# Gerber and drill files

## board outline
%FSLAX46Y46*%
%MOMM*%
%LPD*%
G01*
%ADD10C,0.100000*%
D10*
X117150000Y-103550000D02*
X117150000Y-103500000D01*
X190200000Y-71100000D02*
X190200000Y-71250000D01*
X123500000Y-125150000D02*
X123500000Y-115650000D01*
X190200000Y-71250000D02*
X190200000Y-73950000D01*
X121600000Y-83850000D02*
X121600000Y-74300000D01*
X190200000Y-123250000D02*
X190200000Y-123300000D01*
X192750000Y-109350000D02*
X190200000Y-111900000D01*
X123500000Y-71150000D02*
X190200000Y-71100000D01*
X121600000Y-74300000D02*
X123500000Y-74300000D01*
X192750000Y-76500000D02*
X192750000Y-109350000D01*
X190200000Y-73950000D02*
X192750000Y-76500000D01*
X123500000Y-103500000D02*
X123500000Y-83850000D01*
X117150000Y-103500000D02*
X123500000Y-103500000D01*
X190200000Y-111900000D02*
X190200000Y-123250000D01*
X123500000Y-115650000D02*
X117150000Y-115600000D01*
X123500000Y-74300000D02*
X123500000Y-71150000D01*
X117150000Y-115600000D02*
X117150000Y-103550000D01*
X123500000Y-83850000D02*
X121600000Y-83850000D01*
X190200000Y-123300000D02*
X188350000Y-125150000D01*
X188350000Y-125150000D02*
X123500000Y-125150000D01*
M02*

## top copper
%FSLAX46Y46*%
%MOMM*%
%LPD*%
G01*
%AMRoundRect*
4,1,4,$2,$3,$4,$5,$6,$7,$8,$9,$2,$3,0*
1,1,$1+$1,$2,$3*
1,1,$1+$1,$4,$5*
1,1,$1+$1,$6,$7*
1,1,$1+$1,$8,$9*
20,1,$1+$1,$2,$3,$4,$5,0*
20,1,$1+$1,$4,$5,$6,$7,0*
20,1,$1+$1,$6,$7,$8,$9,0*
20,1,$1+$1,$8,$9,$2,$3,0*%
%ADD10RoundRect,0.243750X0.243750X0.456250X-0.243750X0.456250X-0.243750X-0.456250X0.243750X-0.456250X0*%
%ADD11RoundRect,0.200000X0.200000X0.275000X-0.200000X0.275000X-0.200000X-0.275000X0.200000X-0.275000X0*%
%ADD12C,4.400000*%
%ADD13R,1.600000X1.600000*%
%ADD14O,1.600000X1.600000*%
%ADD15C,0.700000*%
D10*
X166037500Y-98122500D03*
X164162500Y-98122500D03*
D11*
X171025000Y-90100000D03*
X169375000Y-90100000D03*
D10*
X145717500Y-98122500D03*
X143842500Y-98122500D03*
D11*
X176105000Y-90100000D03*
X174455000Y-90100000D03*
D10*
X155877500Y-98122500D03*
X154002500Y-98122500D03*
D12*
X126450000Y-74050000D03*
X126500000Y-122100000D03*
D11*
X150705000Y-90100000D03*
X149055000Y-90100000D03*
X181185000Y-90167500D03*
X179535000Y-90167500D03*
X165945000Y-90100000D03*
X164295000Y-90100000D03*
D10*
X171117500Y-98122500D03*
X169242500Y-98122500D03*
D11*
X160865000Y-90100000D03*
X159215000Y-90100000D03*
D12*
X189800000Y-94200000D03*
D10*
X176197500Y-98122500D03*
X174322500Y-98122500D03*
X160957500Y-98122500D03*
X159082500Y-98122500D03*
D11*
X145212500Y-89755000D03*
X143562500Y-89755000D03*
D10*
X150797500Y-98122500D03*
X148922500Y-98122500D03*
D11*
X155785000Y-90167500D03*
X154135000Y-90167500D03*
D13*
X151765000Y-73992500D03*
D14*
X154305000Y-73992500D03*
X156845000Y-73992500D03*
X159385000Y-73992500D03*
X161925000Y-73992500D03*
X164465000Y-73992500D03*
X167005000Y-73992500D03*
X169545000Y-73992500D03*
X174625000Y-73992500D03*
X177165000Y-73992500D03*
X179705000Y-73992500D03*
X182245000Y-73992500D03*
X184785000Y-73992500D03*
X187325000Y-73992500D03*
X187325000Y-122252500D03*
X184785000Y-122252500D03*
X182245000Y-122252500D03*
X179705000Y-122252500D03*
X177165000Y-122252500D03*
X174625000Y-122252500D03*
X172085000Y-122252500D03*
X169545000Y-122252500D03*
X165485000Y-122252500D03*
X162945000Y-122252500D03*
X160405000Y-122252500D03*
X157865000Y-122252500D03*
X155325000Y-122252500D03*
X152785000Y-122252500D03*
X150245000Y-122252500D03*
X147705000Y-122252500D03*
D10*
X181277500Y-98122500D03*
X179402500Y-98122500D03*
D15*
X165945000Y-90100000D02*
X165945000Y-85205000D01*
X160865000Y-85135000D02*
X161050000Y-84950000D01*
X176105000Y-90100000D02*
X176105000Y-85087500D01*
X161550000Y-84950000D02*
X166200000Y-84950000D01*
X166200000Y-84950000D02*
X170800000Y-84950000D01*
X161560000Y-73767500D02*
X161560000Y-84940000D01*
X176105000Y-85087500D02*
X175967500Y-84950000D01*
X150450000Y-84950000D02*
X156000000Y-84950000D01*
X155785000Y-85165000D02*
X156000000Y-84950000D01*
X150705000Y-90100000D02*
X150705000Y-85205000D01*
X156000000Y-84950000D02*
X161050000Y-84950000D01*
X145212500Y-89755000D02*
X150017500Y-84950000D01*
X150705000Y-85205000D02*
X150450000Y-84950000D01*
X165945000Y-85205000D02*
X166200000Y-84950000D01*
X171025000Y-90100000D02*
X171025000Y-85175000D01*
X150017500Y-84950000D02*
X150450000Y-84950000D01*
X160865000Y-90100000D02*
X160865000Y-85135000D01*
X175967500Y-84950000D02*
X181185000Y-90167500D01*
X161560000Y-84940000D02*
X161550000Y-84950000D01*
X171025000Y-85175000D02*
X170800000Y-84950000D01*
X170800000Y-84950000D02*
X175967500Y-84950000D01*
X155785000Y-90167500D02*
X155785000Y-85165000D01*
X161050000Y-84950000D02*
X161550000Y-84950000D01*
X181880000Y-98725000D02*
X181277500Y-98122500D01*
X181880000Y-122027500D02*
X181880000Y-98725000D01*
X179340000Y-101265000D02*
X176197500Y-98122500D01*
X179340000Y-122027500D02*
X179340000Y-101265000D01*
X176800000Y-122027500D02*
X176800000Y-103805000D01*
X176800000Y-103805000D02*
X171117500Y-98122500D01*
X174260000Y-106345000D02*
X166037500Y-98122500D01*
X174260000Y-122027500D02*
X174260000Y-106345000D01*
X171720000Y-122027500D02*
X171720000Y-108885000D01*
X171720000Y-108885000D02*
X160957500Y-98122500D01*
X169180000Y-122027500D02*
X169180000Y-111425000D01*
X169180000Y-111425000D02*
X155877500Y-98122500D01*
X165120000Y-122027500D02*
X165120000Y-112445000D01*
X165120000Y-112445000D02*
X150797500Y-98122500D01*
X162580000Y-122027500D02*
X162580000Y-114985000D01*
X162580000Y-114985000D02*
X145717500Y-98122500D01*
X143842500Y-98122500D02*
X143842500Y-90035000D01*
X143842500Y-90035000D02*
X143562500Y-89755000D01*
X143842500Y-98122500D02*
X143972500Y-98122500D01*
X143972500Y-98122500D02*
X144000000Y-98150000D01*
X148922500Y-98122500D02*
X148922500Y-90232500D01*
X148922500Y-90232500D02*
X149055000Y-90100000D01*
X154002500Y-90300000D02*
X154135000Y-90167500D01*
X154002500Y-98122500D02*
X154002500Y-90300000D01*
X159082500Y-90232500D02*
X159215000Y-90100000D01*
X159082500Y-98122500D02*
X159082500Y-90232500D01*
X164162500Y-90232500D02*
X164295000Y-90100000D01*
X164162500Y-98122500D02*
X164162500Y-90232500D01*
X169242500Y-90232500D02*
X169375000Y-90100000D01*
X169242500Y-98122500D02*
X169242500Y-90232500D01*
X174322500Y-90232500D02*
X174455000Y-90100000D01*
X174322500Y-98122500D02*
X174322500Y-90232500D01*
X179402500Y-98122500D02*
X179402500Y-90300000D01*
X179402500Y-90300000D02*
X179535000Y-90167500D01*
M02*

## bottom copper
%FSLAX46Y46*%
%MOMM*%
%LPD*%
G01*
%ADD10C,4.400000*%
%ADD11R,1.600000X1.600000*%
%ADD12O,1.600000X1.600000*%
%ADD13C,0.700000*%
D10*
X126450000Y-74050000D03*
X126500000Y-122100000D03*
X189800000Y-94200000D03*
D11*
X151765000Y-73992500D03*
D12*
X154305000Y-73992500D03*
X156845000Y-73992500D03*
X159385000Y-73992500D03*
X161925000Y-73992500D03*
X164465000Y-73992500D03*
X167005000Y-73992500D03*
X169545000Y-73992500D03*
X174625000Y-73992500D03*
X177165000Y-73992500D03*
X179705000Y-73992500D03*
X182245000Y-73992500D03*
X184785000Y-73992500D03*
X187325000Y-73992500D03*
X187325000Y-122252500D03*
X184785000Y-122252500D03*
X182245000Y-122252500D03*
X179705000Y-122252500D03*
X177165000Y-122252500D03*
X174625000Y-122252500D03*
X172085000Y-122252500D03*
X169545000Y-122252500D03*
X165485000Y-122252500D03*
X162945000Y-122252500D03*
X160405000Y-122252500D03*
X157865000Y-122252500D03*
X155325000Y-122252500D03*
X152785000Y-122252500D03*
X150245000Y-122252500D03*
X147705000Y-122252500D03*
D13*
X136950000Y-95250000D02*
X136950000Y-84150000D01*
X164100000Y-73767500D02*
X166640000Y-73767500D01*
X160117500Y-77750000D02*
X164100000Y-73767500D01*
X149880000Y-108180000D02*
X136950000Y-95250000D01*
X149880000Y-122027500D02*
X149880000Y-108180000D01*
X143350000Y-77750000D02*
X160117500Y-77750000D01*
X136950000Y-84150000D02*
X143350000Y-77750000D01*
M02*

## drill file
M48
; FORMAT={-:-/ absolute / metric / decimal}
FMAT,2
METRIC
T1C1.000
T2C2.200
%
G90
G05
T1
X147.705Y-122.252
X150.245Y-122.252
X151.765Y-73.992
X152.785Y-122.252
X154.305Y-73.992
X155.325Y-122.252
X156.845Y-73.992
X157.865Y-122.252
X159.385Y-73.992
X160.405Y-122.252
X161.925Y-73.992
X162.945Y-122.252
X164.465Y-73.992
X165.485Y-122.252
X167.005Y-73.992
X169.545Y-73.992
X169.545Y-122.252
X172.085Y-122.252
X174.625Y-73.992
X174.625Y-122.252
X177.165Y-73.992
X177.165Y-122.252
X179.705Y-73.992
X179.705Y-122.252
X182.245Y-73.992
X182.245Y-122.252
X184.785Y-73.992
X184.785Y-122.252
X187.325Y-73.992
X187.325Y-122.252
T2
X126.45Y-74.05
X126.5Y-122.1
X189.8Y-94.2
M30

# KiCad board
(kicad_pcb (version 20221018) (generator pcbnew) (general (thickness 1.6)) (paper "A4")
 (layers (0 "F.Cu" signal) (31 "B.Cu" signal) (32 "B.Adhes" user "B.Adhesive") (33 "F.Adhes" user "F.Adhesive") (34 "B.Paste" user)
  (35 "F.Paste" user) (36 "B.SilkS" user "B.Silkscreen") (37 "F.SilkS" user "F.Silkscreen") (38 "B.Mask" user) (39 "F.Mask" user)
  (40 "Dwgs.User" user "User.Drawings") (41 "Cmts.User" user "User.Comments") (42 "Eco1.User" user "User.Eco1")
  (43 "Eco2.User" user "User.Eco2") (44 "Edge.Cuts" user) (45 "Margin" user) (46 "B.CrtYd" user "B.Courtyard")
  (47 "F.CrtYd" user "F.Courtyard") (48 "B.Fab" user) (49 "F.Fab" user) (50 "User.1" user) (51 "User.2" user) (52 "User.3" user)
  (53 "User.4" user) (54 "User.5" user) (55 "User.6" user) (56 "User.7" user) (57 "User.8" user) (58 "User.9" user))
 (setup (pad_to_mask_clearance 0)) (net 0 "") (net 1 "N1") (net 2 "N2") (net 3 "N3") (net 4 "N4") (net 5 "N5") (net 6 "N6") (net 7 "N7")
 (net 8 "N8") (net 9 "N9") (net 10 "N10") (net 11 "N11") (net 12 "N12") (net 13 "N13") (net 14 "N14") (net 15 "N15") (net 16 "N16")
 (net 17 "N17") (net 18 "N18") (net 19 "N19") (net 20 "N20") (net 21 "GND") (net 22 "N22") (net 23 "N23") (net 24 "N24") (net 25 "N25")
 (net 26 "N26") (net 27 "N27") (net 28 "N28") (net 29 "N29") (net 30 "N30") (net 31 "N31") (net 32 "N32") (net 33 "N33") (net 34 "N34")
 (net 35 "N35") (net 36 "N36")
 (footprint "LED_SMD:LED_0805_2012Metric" (layer "F.Cu") (at 165.1 98.1225 180)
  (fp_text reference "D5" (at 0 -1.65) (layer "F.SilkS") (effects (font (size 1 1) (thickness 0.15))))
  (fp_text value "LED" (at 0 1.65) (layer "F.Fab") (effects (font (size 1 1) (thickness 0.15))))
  (pad "1" smd roundrect (at -0.9375 0 180) (size 0.975 1.4) (layers "F.Cu" "F.Paste" "F.Mask") (roundrect_rratio 0.25) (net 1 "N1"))
  (pad "2" smd roundrect (at 0.9375 0 180) (size 0.975 1.4) (layers "F.Cu" "F.Paste" "F.Mask") (roundrect_rratio 0.25) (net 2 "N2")))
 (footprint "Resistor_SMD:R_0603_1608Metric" (layer "F.Cu") (at 170.2 90.1 180)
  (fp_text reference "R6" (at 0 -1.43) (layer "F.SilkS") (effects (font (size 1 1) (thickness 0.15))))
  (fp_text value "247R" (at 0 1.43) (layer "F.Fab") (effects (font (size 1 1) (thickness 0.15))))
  (pad "1" smd roundrect (at -0.825 0 180) (size 0.8 0.95) (layers "F.Cu" "F.Paste" "F.Mask") (roundrect_rratio 0.25) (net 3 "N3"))
  (pad "2" smd roundrect (at 0.825 0 180) (size 0.8 0.95) (layers "F.Cu" "F.Paste" "F.Mask") (roundrect_rratio 0.25) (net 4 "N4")))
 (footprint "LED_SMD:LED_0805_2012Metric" (layer "F.Cu") (at 144.78 98.1225 180)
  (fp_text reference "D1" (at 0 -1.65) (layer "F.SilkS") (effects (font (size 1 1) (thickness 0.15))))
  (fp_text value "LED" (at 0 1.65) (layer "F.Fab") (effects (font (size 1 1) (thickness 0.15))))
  (pad "1" smd roundrect (at -0.9375 0 180) (size 0.975 1.4) (layers "F.Cu" "F.Paste" "F.Mask") (roundrect_rratio 0.25) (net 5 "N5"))
  (pad "2" smd roundrect (at 0.9375 0 180) (size 0.975 1.4) (layers "F.Cu" "F.Paste" "F.Mask") (roundrect_rratio 0.25) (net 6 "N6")))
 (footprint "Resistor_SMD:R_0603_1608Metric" (layer "F.Cu") (at 175.28 90.1 180)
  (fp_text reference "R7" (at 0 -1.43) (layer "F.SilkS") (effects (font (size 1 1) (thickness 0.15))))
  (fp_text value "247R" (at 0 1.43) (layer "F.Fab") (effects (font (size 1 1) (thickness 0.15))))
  (pad "1" smd roundrect (at -0.825 0 180) (size 0.8 0.95) (layers "F.Cu" "F.Paste" "F.Mask") (roundrect_rratio 0.25) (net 3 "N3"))
  (pad "2" smd roundrect (at 0.825 0 180) (size 0.8 0.95) (layers "F.Cu" "F.Paste" "F.Mask") (roundrect_rratio 0.25) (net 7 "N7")))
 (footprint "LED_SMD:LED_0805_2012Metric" (layer "F.Cu") (at 154.94 98.1225 180)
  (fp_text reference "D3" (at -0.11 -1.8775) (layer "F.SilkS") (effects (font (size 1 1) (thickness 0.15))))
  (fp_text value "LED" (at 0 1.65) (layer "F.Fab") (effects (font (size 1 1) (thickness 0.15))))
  (pad "1" smd roundrect (at -0.9375 0 180) (size 0.975 1.4) (layers "F.Cu" "F.Paste" "F.Mask") (roundrect_rratio 0.25) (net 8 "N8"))
  (pad "2" smd roundrect (at 0.9375 0 180) (size 0.975 1.4) (layers "F.Cu" "F.Paste" "F.Mask") (roundrect_rratio 0.25) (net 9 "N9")))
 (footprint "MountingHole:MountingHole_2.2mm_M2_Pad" (layer "F.Cu") (at 126.45 74.05)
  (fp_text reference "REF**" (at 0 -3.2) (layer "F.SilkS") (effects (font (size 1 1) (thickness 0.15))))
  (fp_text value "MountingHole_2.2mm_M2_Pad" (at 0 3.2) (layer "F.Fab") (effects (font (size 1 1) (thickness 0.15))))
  (pad "1" thru_hole circle (at 0 0) (size 4.4 4.4) (drill 2.2) (layers "*.Cu" "*.Mask")))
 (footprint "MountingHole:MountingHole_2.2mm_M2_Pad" (layer "F.Cu") (at 126.5 122.1)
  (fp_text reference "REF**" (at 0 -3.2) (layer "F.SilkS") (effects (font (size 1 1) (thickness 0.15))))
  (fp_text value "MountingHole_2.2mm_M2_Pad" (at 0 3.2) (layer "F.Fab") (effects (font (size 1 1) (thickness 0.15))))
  (pad "1" thru_hole circle (at 0 0) (size 4.4 4.4) (drill 2.2) (layers "*.Cu" "*.Mask")))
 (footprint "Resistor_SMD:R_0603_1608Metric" (layer "F.Cu") (at 149.88 90.1 180)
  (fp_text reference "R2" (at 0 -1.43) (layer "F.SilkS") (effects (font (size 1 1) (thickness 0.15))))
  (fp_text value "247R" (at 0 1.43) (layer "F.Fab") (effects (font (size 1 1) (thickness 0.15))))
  (pad "1" smd roundrect (at -0.825 0 180) (size 0.8 0.95) (layers "F.Cu" "F.Paste" "F.Mask") (roundrect_rratio 0.25) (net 3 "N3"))
  (pad "2" smd roundrect (at 0.825 0 180) (size 0.8 0.95) (layers "F.Cu" "F.Paste" "F.Mask") (roundrect_rratio 0.25) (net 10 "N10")))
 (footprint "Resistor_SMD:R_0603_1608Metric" (layer "F.Cu") (at 180.36 90.1675 180)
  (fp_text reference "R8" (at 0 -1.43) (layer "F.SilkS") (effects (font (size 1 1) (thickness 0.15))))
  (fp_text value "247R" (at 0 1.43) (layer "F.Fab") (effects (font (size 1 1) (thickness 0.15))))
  (pad "1" smd roundrect (at -0.825 0 180) (size 0.8 0.95) (layers "F.Cu" "F.Paste" "F.Mask") (roundrect_rratio 0.25) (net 3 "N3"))
  (pad "2" smd roundrect (at 0.825 0 180) (size 0.8 0.95) (layers "F.Cu" "F.Paste" "F.Mask") (roundrect_rratio 0.25) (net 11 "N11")))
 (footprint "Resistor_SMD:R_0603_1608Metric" (layer "F.Cu") (at 165.12 90.1 180)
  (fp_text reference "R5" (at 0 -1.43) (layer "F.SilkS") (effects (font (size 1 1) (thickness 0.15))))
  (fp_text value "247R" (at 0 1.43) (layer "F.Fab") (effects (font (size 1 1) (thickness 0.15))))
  (pad "1" smd roundrect (at -0.825 0 180) (size 0.8 0.95) (layers "F.Cu" "F.Paste" "F.Mask") (roundrect_rratio 0.25) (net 3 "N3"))
  (pad "2" smd roundrect (at 0.825 0 180) (size 0.8 0.95) (layers "F.Cu" "F.Paste" "F.Mask") (roundrect_rratio 0.25) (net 2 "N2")))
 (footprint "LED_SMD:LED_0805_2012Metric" (layer "F.Cu") (at 170.18 98.1225 180)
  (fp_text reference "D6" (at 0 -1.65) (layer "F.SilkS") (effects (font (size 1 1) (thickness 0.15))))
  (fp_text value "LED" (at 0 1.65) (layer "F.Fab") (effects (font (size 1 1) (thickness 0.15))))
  (pad "1" smd roundrect (at -0.9375 0 180) (size 0.975 1.4) (layers "F.Cu" "F.Paste" "F.Mask") (roundrect_rratio 0.25) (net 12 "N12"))
  (pad "2" smd roundrect (at 0.9375 0 180) (size 0.975 1.4) (layers "F.Cu" "F.Paste" "F.Mask") (roundrect_rratio 0.25) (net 4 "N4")))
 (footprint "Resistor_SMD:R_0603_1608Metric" (layer "F.Cu") (at 160.04 90.1 180)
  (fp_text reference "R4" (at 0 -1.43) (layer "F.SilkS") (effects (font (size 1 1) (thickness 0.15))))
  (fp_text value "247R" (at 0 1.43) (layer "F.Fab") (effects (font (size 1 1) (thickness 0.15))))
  (pad "1" smd roundrect (at -0.825 0 180) (size 0.8 0.95) (layers "F.Cu" "F.Paste" "F.Mask") (roundrect_rratio 0.25) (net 3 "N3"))
  (pad "2" smd roundrect (at 0.825 0 180) (size 0.8 0.95) (layers "F.Cu" "F.Paste" "F.Mask") (roundrect_rratio 0.25) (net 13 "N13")))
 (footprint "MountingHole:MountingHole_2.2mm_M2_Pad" (layer "F.Cu") (at 189.8 94.2)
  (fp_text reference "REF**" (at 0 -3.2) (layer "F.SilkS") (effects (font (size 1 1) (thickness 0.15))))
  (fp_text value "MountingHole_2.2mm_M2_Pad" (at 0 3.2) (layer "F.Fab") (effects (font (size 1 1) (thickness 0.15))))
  (pad "1" thru_hole circle (at 0 0) (size 4.4 4.4) (drill 2.2) (layers "*.Cu" "*.Mask")))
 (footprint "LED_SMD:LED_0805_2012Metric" (layer "F.Cu") (at 175.26 98.1225 180)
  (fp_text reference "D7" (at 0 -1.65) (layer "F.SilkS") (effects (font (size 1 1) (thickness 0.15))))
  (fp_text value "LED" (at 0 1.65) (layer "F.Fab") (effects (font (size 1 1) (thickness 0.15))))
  (pad "1" smd roundrect (at -0.9375 0 180) (size 0.975 1.4) (layers "F.Cu" "F.Paste" "F.Mask") (roundrect_rratio 0.25) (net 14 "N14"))
  (pad "2" smd roundrect (at 0.9375 0 180) (size 0.975 1.4) (layers "F.Cu" "F.Paste" "F.Mask") (roundrect_rratio 0.25) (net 7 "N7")))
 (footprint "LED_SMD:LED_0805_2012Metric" (layer "F.Cu") (at 160.02 98.1225 180)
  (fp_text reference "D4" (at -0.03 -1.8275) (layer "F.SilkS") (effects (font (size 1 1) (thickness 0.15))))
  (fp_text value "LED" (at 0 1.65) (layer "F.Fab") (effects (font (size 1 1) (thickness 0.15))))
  (pad "1" smd roundrect (at -0.9375 0 180) (size 0.975 1.4) (layers "F.Cu" "F.Paste" "F.Mask") (roundrect_rratio 0.25) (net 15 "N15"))
  (pad "2" smd roundrect (at 0.9375 0 180) (size 0.975 1.4) (layers "F.Cu" "F.Paste" "F.Mask") (roundrect_rratio 0.25) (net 13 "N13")))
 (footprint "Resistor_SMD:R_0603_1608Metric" (layer "F.Cu") (at 144.3875 89.755 180)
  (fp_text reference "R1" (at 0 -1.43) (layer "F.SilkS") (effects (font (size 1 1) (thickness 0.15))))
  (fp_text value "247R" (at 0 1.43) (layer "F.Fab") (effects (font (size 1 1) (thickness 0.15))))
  (pad "1" smd roundrect (at -0.825 0 180) (size 0.8 0.95) (layers "F.Cu" "F.Paste" "F.Mask") (roundrect_rratio 0.25) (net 3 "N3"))
  (pad "2" smd roundrect (at 0.825 0 180) (size 0.8 0.95) (layers "F.Cu" "F.Paste" "F.Mask") (roundrect_rratio 0.25) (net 6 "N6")))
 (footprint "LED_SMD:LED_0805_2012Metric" (layer "F.Cu") (at 149.86 98.1225 180)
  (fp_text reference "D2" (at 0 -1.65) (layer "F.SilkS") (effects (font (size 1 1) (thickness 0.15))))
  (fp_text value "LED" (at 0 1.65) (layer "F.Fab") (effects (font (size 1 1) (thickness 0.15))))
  (pad "1" smd roundrect (at -0.9375 0 180) (size 0.975 1.4) (layers "F.Cu" "F.Paste" "F.Mask") (roundrect_rratio 0.25) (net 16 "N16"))
  (pad "2" smd roundrect (at 0.9375 0 180) (size 0.975 1.4) (layers "F.Cu" "F.Paste" "F.Mask") (roundrect_rratio 0.25) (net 10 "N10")))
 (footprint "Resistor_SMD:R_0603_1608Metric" (layer "F.Cu") (at 154.96 90.1675 180)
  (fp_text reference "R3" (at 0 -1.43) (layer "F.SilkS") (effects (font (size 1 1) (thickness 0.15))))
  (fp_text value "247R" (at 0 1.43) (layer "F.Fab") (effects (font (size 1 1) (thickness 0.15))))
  (pad "1" smd roundrect (at -0.825 0 180) (size 0.8 0.95) (layers "F.Cu" "F.Paste" "F.Mask") (roundrect_rratio 0.25) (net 3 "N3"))
  (pad "2" smd roundrect (at 0.825 0 180) (size 0.8 0.95) (layers "F.Cu" "F.Paste" "F.Mask") (roundrect_rratio 0.25) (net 9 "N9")))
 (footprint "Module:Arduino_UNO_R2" (layer "F.Cu") (at 151.765 73.9925)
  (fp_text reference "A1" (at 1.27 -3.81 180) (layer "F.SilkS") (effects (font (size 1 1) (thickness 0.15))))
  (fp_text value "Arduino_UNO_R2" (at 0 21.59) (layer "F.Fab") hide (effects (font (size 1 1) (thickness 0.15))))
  (pad "1" thru_hole rect (at 0 0 90) (size 1.6 1.6) (drill 1) (layers "*.Cu" "*.Mask") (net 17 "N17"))
  (pad "2" thru_hole oval (at 2.54 0 90) (size 1.6 1.6) (drill 1) (layers "*.Cu" "*.Mask") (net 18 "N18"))
  (pad "3" thru_hole oval (at 5.08 0 90) (size 1.6 1.6) (drill 1) (layers "*.Cu" "*.Mask") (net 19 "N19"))
  (pad "4" thru_hole oval (at 7.62 0 90) (size 1.6 1.6) (drill 1) (layers "*.Cu" "*.Mask") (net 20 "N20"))
  (pad "5" thru_hole oval (at 10.16 0 90) (size 1.6 1.6) (drill 1) (layers "*.Cu" "*.Mask") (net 3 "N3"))
  (pad "6" thru_hole oval (at 12.7 0 90) (size 1.6 1.6) (drill 1) (layers "*.Cu" "*.Mask") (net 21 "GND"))
  (pad "7" thru_hole oval (at 15.24 0 90) (size 1.6 1.6) (drill 1) (layers "*.Cu" "*.Mask") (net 21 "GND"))
  (pad "8" thru_hole oval (at 17.78 0 90) (size 1.6 1.6) (drill 1) (layers "*.Cu" "*.Mask") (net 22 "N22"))
  (pad "9" thru_hole oval (at 22.86 0 90) (size 1.6 1.6) (drill 1) (layers "*.Cu" "*.Mask") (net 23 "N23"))
  (pad "10" thru_hole oval (at 25.4 0 90) (size 1.6 1.6) (drill 1) (layers "*.Cu" "*.Mask") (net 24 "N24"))
  (pad "11" thru_hole oval (at 27.94 0 90) (size 1.6 1.6) (drill 1) (layers "*.Cu" "*.Mask") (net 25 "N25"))
  (pad "12" thru_hole oval (at 30.48 0 90) (size 1.6 1.6) (drill 1) (layers "*.Cu" "*.Mask") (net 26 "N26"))
  (pad "13" thru_hole oval (at 33.02 0 90) (size 1.6 1.6) (drill 1) (layers "*.Cu" "*.Mask") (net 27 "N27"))
  (pad "14" thru_hole oval (at 35.56 0 90) (size 1.6 1.6) (drill 1) (layers "*.Cu" "*.Mask") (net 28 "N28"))
  (pad "15" thru_hole oval (at 35.56 48.26 90) (size 1.6 1.6) (drill 1) (layers "*.Cu" "*.Mask") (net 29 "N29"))
  (pad "16" thru_hole oval (at 33.02 48.26 90) (size 1.6 1.6) (drill 1) (layers "*.Cu" "*.Mask") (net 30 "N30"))
  (pad "17" thru_hole oval (at 30.48 48.26 90) (size 1.6 1.6) (drill 1) (layers "*.Cu" "*.Mask") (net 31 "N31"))
  (pad "18" thru_hole oval (at 27.94 48.26 90) (size 1.6 1.6) (drill 1) (layers "*.Cu" "*.Mask") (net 14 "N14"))
  (pad "19" thru_hole oval (at 25.4 48.26 90) (size 1.6 1.6) (drill 1) (layers "*.Cu" "*.Mask") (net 12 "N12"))
  (pad "20" thru_hole oval (at 22.86 48.26 90) (size 1.6 1.6) (drill 1) (layers "*.Cu" "*.Mask") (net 1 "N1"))
  (pad "21" thru_hole oval (at 20.32 48.26 90) (size 1.6 1.6) (drill 1) (layers "*.Cu" "*.Mask") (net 15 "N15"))
  (pad "22" thru_hole oval (at 17.78 48.26 90) (size 1.6 1.6) (drill 1) (layers "*.Cu" "*.Mask") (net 8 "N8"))
  (pad "23" thru_hole oval (at 13.72 48.26 90) (size 1.6 1.6) (drill 1) (layers "*.Cu" "*.Mask") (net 16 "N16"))
  (pad "24" thru_hole oval (at 11.18 48.26 90) (size 1.6 1.6) (drill 1) (layers "*.Cu" "*.Mask") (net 5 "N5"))
  (pad "25" thru_hole oval (at 8.64 48.26 90) (size 1.6 1.6) (drill 1) (layers "*.Cu" "*.Mask") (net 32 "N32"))
  (pad "26" thru_hole oval (at 6.1 48.26 90) (size 1.6 1.6) (drill 1) (layers "*.Cu" "*.Mask") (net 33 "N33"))
  (pad "27" thru_hole oval (at 3.56 48.26 90) (size 1.6 1.6) (drill 1) (layers "*.Cu" "*.Mask") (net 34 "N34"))
  (pad "28" thru_hole oval (at 1.02 48.26 90) (size 1.6 1.6) (drill 1) (layers "*.Cu" "*.Mask") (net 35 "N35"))
  (pad "29" thru_hole oval (at -1.52 48.26 90) (size 1.6 1.6) (drill 1) (layers "*.Cu" "*.Mask") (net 21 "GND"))
  (pad "30" thru_hole oval (at -4.06 48.26 90) (size 1.6 1.6) (drill 1) (layers "*.Cu" "*.Mask") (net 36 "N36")))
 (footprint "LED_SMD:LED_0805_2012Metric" (layer "F.Cu") (at 180.34 98.1225 180)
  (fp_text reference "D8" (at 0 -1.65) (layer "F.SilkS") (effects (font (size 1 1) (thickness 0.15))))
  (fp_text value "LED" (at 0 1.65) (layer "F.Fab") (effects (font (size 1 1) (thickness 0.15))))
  (pad "1" smd roundrect (at -0.9375 0 180) (size 0.975 1.4) (layers "F.Cu" "F.Paste" "F.Mask") (roundrect_rratio 0.25) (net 31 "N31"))
  (pad "2" smd roundrect (at 0.9375 0 180) (size 0.975 1.4) (layers "F.Cu" "F.Paste" "F.Mask") (roundrect_rratio 0.25) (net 11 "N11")))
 (gr_line (start 117.15 103.55) (end 117.15 103.5) (stroke (width 0.1) (type default)) (layer "Edge.Cuts"))
 (gr_line (start 190.2 71.1) (end 190.2 71.25) (stroke (width 0.1) (type default)) (layer "Edge.Cuts"))
 (gr_line (start 123.5 125.15) (end 123.5 115.65) (stroke (width 0.1) (type default)) (layer "Edge.Cuts"))
 (gr_line (start 190.2 71.25) (end 190.2 73.95) (stroke (width 0.1) (type default)) (layer "Edge.Cuts"))
 (gr_line (start 121.6 83.85) (end 121.6 74.3) (stroke (width 0.1) (type default)) (layer "Edge.Cuts"))
 (gr_line (start 190.2 123.25) (end 190.2 123.3) (stroke (width 0.1) (type default)) (layer "Edge.Cuts"))
 (gr_line (start 192.75 109.35) (end 190.2 111.9) (stroke (width 0.1) (type default)) (layer "Edge.Cuts"))
 (gr_line (start 123.5 71.15) (end 190.2 71.1) (stroke (width 0.1) (type default)) (layer "Edge.Cuts"))
 (gr_line (start 121.6 74.3) (end 123.5 74.3) (stroke (width 0.1) (type default)) (layer "Edge.Cuts"))
 (gr_line (start 192.75 76.5) (end 192.75 109.35) (stroke (width 0.1) (type default)) (layer "Edge.Cuts"))
 (gr_line (start 190.2 73.95) (end 192.75 76.5) (stroke (width 0.1) (type default)) (layer "Edge.Cuts"))
 (gr_line (start 123.5 103.5) (end 123.5 83.85) (stroke (width 0.1) (type default)) (layer "Edge.Cuts"))
 (gr_line (start 117.15 103.5) (end 123.5 103.5) (stroke (width 0.1) (type default)) (layer "Edge.Cuts"))
 (gr_line (start 190.2 111.9) (end 190.2 123.25) (stroke (width 0.1) (type default)) (layer "Edge.Cuts"))
 (gr_line (start 123.5 115.65) (end 117.15 115.6) (stroke (width 0.1) (type default)) (layer "Edge.Cuts"))
 (gr_line (start 123.5 74.3) (end 123.5 71.15) (stroke (width 0.1) (type default)) (layer "Edge.Cuts"))
 (gr_line (start 117.15 115.6) (end 117.15 103.55) (stroke (width 0.1) (type default)) (layer "Edge.Cuts"))
 (gr_line (start 123.5 83.85) (end 121.6 83.85) (stroke (width 0.1) (type default)) (layer "Edge.Cuts"))
 (gr_line (start 190.2 123.3) (end 188.35 125.15) (stroke (width 0.1) (type default)) (layer "Edge.Cuts"))
 (gr_line (start 188.35 125.15) (end 123.5 125.15) (stroke (width 0.1) (type default)) (layer "Edge.Cuts"))
 (segment (start 165.945 90.1) (end 165.945 85.205) (width 0.7) (layer "F.Cu") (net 3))
 (segment (start 160.865 85.135) (end 161.05 84.95) (width 0.7) (layer "F.Cu") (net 3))
 (segment (start 176.105 90.1) (end 176.105 85.0875) (width 0.7) (layer "F.Cu") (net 3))
 (segment (start 161.55 84.95) (end 166.2 84.95) (width 0.7) (layer "F.Cu") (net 3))
 (segment (start 166.2 84.95) (end 170.8 84.95) (width 0.7) (layer "F.Cu") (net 3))
 (segment (start 161.56 73.7675) (end 161.56 84.94) (width 0.7) (layer "F.Cu") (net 3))
 (segment (start 176.105 85.0875) (end 175.9675 84.95) (width 0.7) (layer "F.Cu") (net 3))
 (segment (start 150.45 84.95) (end 156 84.95) (width 0.7) (layer "F.Cu") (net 3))
 (segment (start 155.785 85.165) (end 156 84.95) (width 0.7) (layer "F.Cu") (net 3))
 (segment (start 150.705 90.1) (end 150.705 85.205) (width 0.7) (layer "F.Cu") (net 3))
 (segment (start 156 84.95) (end 161.05 84.95) (width 0.7) (layer "F.Cu") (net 3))
 (segment (start 145.2125 89.755) (end 150.0175 84.95) (width 0.7) (layer "F.Cu") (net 3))
 (segment (start 150.705 85.205) (end 150.45 84.95) (width 0.7) (layer "F.Cu") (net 3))
 (segment (start 165.945 85.205) (end 166.2 84.95) (width 0.7) (layer "F.Cu") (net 3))
 (segment (start 171.025 90.1) (end 171.025 85.175) (width 0.7) (layer "F.Cu") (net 3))
 (segment (start 150.0175 84.95) (end 150.45 84.95) (width 0.7) (layer "F.Cu") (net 3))
 (segment (start 160.865 90.1) (end 160.865 85.135) (width 0.7) (layer "F.Cu") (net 3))
 (segment (start 175.9675 84.95) (end 181.185 90.1675) (width 0.7) (layer "F.Cu") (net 3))
 (segment (start 161.56 84.94) (end 161.55 84.95) (width 0.7) (layer "F.Cu") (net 3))
 (segment (start 171.025 85.175) (end 170.8 84.95) (width 0.7) (layer "F.Cu") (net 3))
 (segment (start 170.8 84.95) (end 175.9675 84.95) (width 0.7) (layer "F.Cu") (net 3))
 (segment (start 155.785 90.1675) (end 155.785 85.165) (width 0.7) (layer "F.Cu") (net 3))
 (segment (start 161.05 84.95) (end 161.55 84.95) (width 0.7) (layer "F.Cu") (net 3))
 (segment (start 136.95 95.25) (end 136.95 84.15) (width 0.7) (layer "B.Cu") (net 21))
 (segment (start 164.1 73.7675) (end 166.64 73.7675) (width 0.7) (layer "B.Cu") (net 21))
 (segment (start 160.1175 77.75) (end 164.1 73.7675) (width 0.7) (layer "B.Cu") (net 21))
 (segment (start 149.88 108.18) (end 136.95 95.25) (width 0.7) (layer "B.Cu") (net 21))
 (segment (start 149.88 122.0275) (end 149.88 108.18) (width 0.7) (layer "B.Cu") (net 21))
 (segment (start 143.35 77.75) (end 160.1175 77.75) (width 0.7) (layer "B.Cu") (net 21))
 (segment (start 136.95 84.15) (end 143.35 77.75) (width 0.7) (layer "B.Cu") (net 21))
 (segment (start 181.88 98.725) (end 181.2775 98.1225) (width 0.7) (layer "F.Cu") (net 31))
 (segment (start 181.88 122.0275) (end 181.88 98.725) (width 0.7) (layer "F.Cu") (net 31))
 (segment (start 179.34 101.265) (end 176.1975 98.1225) (width 0.7) (layer "F.Cu") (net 14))
 (segment (start 179.34 122.0275) (end 179.34 101.265) (width 0.7) (layer "F.Cu") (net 14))
 (segment (start 176.8 122.0275) (end 176.8 103.805) (width 0.7) (layer "F.Cu") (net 12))
 (segment (start 176.8 103.805) (end 171.1175 98.1225) (width 0.7) (layer "F.Cu") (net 12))
 (segment (start 174.26 106.345) (end 166.0375 98.1225) (width 0.7) (layer "F.Cu") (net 1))
 (segment (start 174.26 122.0275) (end 174.26 106.345) (width 0.7) (layer "F.Cu") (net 1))
 (segment (start 171.72 122.0275) (end 171.72 108.885) (width 0.7) (layer "F.Cu") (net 15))
 (segment (start 171.72 108.885) (end 160.9575 98.1225) (width 0.7) (layer "F.Cu") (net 15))
 (segment (start 169.18 122.0275) (end 169.18 111.425) (width 0.7) (layer "F.Cu") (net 8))
 (segment (start 169.18 111.425) (end 155.8775 98.1225) (width 0.7) (layer "F.Cu") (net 8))
 (segment (start 165.12 122.0275) (end 165.12 112.445) (width 0.7) (layer "F.Cu") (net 16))
 (segment (start 165.12 112.445) (end 150.7975 98.1225) (width 0.7) (layer "F.Cu") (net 16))
 (segment (start 162.58 122.0275) (end 162.58 114.985) (width 0.7) (layer "F.Cu") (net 5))
 (segment (start 162.58 114.985) (end 145.7175 98.1225) (width 0.7) (layer "F.Cu") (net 5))
 (segment (start 143.8425 98.1225) (end 143.8425 90.035) (width 0.7) (layer "F.Cu") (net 6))
 (segment (start 143.8425 90.035) (end 143.5625 89.755) (width 0.7) (layer "F.Cu") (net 6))
 (segment (start 143.8425 98.1225) (end 143.9725 98.1225) (width 0.7) (layer "F.Cu") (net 6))
 (segment (start 143.9725 98.1225) (end 144 98.15) (width 0.7) (layer "F.Cu") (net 6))
 (segment (start 148.9225 98.1225) (end 148.9225 90.2325) (width 0.7) (layer "F.Cu") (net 10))
 (segment (start 148.9225 90.2325) (end 149.055 90.1) (width 0.7) (layer "F.Cu") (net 10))
 (segment (start 154.0025 90.3) (end 154.135 90.1675) (width 0.7) (layer "F.Cu") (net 9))
 (segment (start 154.0025 98.1225) (end 154.0025 90.3) (width 0.7) (layer "F.Cu") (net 9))
 (segment (start 159.0825 90.2325) (end 159.215 90.1) (width 0.7) (layer "F.Cu") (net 13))
 (segment (start 159.0825 98.1225) (end 159.0825 90.2325) (width 0.7) (layer "F.Cu") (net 13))
 (segment (start 164.1625 90.2325) (end 164.295 90.1) (width 0.7) (layer "F.Cu") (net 2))
 (segment (start 164.1625 98.1225) (end 164.1625 90.2325) (width 0.7) (layer "F.Cu") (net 2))
 (segment (start 169.2425 90.2325) (end 169.375 90.1) (width 0.7) (layer "F.Cu") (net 4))
 (segment (start 169.2425 98.1225) (end 169.2425 90.2325) (width 0.7) (layer "F.Cu") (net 4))
 (segment (start 174.3225 90.2325) (end 174.455 90.1) (width 0.7) (layer "F.Cu") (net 7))
 (segment (start 174.3225 98.1225) (end 174.3225 90.2325) (width 0.7) (layer "F.Cu") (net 7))
 (segment (start 179.4025 98.1225) (end 179.4025 90.3) (width 0.7) (layer "F.Cu") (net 11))
 (segment (start 179.4025 90.3) (end 179.535 90.1675) (width 0.7) (layer "F.Cu") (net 11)))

